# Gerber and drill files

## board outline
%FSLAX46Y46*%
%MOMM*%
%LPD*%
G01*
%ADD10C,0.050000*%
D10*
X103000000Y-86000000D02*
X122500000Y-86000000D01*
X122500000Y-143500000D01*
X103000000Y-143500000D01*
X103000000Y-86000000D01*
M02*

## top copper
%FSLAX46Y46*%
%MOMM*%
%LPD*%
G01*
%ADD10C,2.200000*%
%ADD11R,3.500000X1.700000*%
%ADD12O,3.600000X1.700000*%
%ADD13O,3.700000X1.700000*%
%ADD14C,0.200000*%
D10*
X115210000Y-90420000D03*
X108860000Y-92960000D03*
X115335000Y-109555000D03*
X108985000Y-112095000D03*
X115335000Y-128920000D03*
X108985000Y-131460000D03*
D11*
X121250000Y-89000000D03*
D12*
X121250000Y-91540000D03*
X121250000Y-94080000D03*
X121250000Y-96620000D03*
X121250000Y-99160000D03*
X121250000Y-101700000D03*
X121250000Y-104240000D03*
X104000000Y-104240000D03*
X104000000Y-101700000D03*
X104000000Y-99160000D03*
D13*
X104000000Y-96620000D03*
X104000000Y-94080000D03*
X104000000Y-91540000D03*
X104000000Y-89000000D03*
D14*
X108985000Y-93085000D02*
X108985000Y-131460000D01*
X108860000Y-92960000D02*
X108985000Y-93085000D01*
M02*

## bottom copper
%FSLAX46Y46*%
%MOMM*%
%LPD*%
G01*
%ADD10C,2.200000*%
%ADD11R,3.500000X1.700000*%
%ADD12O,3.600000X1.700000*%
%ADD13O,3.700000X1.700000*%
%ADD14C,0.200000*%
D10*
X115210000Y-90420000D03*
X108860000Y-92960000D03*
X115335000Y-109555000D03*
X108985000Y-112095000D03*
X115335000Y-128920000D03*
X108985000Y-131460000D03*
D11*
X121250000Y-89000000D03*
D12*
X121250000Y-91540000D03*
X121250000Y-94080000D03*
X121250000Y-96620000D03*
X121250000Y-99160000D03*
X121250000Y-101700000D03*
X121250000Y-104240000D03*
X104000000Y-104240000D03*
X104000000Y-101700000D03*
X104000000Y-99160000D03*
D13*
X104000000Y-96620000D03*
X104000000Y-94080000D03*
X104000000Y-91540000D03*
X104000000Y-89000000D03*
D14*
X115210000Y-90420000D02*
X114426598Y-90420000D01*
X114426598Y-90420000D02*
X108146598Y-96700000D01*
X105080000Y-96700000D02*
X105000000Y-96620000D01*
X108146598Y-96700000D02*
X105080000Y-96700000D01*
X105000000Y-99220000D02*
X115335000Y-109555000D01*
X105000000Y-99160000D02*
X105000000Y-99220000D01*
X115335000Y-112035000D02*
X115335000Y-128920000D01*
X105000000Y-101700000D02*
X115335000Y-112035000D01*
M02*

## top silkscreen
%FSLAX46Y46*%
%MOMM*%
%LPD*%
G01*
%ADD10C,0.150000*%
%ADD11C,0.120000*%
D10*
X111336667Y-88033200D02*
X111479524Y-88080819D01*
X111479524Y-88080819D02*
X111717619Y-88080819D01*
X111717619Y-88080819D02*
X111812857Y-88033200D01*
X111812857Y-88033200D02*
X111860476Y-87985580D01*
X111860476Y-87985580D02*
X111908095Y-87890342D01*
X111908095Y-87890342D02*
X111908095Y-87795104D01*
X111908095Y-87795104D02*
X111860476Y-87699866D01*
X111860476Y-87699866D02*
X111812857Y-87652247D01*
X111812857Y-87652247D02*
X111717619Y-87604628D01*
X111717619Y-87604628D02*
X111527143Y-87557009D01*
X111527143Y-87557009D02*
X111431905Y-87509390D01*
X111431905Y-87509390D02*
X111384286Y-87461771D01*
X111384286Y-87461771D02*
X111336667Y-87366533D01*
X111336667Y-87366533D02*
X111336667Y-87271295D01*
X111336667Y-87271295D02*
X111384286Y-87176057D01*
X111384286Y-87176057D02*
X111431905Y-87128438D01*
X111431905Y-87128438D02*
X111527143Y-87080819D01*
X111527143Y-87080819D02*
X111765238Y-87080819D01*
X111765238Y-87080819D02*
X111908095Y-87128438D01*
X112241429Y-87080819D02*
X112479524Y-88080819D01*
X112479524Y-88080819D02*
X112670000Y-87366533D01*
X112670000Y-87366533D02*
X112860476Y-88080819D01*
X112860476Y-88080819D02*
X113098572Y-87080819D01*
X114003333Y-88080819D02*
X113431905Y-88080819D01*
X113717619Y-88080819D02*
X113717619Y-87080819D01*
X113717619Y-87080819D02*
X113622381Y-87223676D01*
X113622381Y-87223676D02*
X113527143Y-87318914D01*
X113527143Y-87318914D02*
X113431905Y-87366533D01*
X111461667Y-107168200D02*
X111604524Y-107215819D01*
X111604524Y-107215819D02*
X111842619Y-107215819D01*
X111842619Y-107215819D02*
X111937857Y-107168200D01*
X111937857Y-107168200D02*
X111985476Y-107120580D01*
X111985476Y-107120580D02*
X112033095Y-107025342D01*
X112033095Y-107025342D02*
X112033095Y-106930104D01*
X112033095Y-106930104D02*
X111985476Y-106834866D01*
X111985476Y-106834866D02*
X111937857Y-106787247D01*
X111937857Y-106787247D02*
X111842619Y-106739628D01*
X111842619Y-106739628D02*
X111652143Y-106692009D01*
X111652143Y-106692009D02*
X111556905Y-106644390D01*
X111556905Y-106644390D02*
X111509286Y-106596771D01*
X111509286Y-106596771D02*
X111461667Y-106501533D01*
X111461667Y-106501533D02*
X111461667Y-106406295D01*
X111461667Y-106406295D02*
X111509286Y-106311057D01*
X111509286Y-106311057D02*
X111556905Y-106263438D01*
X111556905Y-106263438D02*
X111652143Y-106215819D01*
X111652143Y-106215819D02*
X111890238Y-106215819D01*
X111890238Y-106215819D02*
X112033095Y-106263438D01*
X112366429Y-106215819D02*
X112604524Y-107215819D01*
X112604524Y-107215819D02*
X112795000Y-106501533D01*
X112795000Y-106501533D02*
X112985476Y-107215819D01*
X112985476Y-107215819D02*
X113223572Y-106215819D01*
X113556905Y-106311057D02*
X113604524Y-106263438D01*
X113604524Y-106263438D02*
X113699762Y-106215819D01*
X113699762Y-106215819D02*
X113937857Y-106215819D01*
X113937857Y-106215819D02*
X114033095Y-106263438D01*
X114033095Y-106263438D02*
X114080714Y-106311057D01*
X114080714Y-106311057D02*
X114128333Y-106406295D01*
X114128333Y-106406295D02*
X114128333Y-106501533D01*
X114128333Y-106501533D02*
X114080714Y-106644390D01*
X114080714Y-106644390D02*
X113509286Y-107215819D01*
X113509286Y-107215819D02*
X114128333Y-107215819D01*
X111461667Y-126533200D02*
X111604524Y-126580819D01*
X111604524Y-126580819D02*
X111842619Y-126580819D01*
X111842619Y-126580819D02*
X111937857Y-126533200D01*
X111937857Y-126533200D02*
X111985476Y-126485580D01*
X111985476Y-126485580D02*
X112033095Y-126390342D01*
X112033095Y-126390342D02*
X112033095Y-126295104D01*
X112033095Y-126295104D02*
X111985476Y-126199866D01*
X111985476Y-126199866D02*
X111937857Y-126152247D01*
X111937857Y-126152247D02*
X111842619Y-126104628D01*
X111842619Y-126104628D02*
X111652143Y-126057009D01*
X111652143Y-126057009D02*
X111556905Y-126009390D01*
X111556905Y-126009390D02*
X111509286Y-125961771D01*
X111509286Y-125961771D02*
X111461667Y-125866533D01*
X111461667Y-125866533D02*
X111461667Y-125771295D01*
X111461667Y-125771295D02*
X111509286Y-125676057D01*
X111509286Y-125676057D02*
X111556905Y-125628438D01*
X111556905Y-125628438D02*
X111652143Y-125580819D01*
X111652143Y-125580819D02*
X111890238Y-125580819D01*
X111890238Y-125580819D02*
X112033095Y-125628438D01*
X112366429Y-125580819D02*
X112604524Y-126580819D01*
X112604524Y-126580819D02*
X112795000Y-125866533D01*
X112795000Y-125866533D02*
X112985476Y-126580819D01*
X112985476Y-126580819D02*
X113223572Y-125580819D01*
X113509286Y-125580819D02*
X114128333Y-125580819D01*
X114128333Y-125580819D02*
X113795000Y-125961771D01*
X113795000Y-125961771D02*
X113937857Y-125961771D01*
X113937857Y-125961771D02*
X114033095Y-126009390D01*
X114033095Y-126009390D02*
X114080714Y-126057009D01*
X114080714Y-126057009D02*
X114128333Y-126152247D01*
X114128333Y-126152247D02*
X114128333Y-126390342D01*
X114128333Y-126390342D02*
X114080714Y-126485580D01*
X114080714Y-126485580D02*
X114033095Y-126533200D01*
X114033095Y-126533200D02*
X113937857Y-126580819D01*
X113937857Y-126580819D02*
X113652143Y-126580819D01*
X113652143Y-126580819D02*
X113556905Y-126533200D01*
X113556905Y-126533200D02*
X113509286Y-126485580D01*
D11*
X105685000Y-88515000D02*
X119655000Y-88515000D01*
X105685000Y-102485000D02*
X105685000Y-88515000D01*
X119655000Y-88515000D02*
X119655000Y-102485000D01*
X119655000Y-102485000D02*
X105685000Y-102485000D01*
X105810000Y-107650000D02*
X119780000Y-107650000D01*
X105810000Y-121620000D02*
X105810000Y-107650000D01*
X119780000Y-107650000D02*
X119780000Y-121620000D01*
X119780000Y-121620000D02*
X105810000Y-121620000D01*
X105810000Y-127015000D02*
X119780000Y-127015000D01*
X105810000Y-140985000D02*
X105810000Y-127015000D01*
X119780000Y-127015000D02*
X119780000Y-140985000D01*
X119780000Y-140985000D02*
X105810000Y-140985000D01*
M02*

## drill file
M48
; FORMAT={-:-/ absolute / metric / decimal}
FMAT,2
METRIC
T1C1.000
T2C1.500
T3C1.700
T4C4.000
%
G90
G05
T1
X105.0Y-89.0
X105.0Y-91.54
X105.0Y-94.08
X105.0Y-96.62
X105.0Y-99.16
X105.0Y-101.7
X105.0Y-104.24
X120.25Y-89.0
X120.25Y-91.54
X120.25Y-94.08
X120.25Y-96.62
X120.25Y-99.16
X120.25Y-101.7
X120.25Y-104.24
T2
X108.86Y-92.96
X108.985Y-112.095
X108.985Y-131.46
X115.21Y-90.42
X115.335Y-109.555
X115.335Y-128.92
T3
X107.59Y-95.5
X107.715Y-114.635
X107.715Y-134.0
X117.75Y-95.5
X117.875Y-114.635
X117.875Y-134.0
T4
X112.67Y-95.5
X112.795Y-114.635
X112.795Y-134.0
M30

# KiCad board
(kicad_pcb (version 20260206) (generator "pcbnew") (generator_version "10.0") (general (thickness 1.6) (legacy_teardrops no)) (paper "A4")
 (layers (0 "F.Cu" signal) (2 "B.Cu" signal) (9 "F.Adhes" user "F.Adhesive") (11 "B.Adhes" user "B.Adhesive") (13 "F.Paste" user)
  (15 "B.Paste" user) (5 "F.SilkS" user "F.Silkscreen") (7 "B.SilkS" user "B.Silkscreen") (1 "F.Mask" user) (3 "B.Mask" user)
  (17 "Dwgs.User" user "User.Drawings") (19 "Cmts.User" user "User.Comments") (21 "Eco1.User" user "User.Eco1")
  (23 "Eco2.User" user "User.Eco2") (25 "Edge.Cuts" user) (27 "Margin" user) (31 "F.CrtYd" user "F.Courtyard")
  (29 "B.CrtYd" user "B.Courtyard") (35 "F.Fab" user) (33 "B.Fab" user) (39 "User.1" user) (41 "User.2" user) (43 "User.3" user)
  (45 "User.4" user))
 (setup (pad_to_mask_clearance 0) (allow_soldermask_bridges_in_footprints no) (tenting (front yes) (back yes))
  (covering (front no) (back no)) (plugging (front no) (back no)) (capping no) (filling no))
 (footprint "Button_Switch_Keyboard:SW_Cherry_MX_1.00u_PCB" (layer "F.Cu") (at 115.21 90.42)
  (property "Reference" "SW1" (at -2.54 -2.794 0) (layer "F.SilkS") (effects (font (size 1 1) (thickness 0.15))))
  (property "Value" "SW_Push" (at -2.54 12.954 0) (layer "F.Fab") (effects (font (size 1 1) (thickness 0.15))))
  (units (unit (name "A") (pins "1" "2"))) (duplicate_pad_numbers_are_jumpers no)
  (fp_line (start -9.525 -1.905) (end 4.445 -1.905) (stroke (width 0.12) (type solid)) (layer "F.SilkS"))
  (fp_line (start -9.525 12.065) (end -9.525 -1.905) (stroke (width 0.12) (type solid)) (layer "F.SilkS"))
  (fp_line (start 4.445 -1.905) (end 4.445 12.065) (stroke (width 0.12) (type solid)) (layer "F.SilkS"))
  (fp_line (start 4.445 12.065) (end -9.525 12.065) (stroke (width 0.12) (type solid)) (layer "F.SilkS"))
  (pad "" np_thru_hole circle (at -7.62 5.08) (size 1.7 1.7) (drill 1.7) (layers "*.Cu" "*.Mask"))
  (pad "" np_thru_hole circle (at -2.54 5.08) (size 4 4) (drill 4) (layers "*.Cu" "*.Mask"))
  (pad "" np_thru_hole circle (at 2.54 5.08) (size 1.7 1.7) (drill 1.7) (layers "*.Cu" "*.Mask"))
  (pad "1" thru_hole circle (at 0 0) (size 2.2 2.2) (drill 1.5) (layers "*.Cu" "*.Mask") (remove_unused_layers no)
   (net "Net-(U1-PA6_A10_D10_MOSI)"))
  (pad "2" thru_hole circle (at -6.35 2.54) (size 2.2 2.2) (drill 1.5) (layers "*.Cu" "*.Mask") (remove_unused_layers no) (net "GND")))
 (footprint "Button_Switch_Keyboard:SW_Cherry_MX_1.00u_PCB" (layer "F.Cu") (at 115.335 109.555)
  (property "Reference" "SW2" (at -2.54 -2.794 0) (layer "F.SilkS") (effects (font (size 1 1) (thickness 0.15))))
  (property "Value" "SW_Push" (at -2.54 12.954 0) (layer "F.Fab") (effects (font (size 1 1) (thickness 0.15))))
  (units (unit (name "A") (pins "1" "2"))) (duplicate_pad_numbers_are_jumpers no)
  (fp_line (start -9.525 -1.905) (end 4.445 -1.905) (stroke (width 0.12) (type solid)) (layer "F.SilkS"))
  (fp_line (start -9.525 12.065) (end -9.525 -1.905) (stroke (width 0.12) (type solid)) (layer "F.SilkS"))
  (fp_line (start 4.445 -1.905) (end 4.445 12.065) (stroke (width 0.12) (type solid)) (layer "F.SilkS"))
  (fp_line (start 4.445 12.065) (end -9.525 12.065) (stroke (width 0.12) (type solid)) (layer "F.SilkS"))
  (pad "" np_thru_hole circle (at -7.62 5.08) (size 1.7 1.7) (drill 1.7) (layers "*.Cu" "*.Mask"))
  (pad "" np_thru_hole circle (at -2.54 5.08) (size 4 4) (drill 4) (layers "*.Cu" "*.Mask"))
  (pad "" np_thru_hole circle (at 2.54 5.08) (size 1.7 1.7) (drill 1.7) (layers "*.Cu" "*.Mask"))
  (pad "1" thru_hole circle (at 0 0) (size 2.2 2.2) (drill 1.5) (layers "*.Cu" "*.Mask") (remove_unused_layers no)
   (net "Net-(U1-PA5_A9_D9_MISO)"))
  (pad "2" thru_hole circle (at -6.35 2.54) (size 2.2 2.2) (drill 1.5) (layers "*.Cu" "*.Mask") (remove_unused_layers no) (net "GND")))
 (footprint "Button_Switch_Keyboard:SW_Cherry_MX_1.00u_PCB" (layer "F.Cu") (at 115.335 128.92)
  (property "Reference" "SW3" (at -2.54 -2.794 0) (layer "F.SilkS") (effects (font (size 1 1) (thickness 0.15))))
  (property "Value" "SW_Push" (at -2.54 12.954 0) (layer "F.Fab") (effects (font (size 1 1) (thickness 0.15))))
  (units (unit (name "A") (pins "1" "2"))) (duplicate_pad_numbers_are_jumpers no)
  (fp_line (start -9.525 -1.905) (end 4.445 -1.905) (stroke (width 0.12) (type solid)) (layer "F.SilkS"))
  (fp_line (start -9.525 12.065) (end -9.525 -1.905) (stroke (width 0.12) (type solid)) (layer "F.SilkS"))
  (fp_line (start 4.445 -1.905) (end 4.445 12.065) (stroke (width 0.12) (type solid)) (layer "F.SilkS"))
  (fp_line (start 4.445 12.065) (end -9.525 12.065) (stroke (width 0.12) (type solid)) (layer "F.SilkS"))
  (pad "" np_thru_hole circle (at -7.62 5.08) (size 1.7 1.7) (drill 1.7) (layers "*.Cu" "*.Mask"))
  (pad "" np_thru_hole circle (at -2.54 5.08) (size 4 4) (drill 4) (layers "*.Cu" "*.Mask"))
  (pad "" np_thru_hole circle (at 2.54 5.08) (size 1.7 1.7) (drill 1.7) (layers "*.Cu" "*.Mask"))
  (pad "1" thru_hole circle (at 0 0) (size 2.2 2.2) (drill 1.5) (layers "*.Cu" "*.Mask") (remove_unused_layers no)
   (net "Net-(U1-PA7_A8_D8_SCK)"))
  (pad "2" thru_hole circle (at -6.35 2.54) (size 2.2 2.2) (drill 1.5) (layers "*.Cu" "*.Mask") (remove_unused_layers no) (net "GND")))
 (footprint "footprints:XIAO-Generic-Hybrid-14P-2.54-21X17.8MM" (layer "B.Cu") (at 112.625 96.62 180)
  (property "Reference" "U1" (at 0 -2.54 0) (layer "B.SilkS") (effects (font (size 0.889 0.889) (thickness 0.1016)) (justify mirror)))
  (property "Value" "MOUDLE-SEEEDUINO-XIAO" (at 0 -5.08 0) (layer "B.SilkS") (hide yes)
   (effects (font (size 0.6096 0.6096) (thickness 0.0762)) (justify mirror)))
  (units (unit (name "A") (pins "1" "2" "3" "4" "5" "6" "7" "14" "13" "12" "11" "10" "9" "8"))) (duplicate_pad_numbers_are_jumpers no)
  (pad "1" thru_hole rect (at -7.625 7.62 180) (size 3.5 1.7) (drill 1 (offset -1 0)) (layers "*.Cu" "*.Mask") (remove_unused_layers no)
   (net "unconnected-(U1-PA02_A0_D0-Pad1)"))
  (pad "2" thru_hole oval (at -7.625 5.08 180) (size 3.6 1.7) (drill 1 (offset -1 0)) (layers "*.Cu" "*.Mask") (remove_unused_layers no)
   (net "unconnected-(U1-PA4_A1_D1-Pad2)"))
  (pad "3" thru_hole oval (at -7.625 2.54 180) (size 3.6 1.7) (drill 1 (offset -1 0)) (layers "*.Cu" "*.Mask") (remove_unused_layers no)
   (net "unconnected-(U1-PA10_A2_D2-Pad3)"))
  (pad "4" thru_hole oval (at -7.625 0 180) (size 3.6 1.7) (drill 1 (offset -1 0)) (layers "*.Cu" "*.Mask") (remove_unused_layers no)
   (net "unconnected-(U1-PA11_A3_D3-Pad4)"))
  (pad "5" thru_hole oval (at -7.625 -2.54 180) (size 3.6 1.7) (drill 1 (offset -1 0)) (layers "*.Cu" "*.Mask") (remove_unused_layers no)
   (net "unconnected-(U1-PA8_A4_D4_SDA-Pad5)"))
  (pad "6" thru_hole oval (at -7.625 -5.08) (size 3.6 1.7) (drill 1 (offset 1 0)) (layers "*.Cu" "*.Mask") (remove_unused_layers no)
   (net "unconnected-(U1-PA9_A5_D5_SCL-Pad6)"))
  (pad "7" thru_hole oval (at -7.625 -7.62 180) (size 3.6 1.7) (drill 1 (offset -1 0)) (layers "*.Cu" "*.Mask") (remove_unused_layers no)
   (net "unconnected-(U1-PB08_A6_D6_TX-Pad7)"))
  (pad "8" thru_hole oval (at 7.625 -7.62 180) (size 3.6 1.7) (drill 1 (offset 1 0)) (layers "*.Cu" "*.Mask") (remove_unused_layers no)
   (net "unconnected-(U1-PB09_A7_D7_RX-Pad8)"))
  (pad "9" thru_hole oval (at 7.625 -5.08 180) (size 3.6 1.7) (drill 1 (offset 1 0)) (layers "*.Cu" "*.Mask") (remove_unused_layers no)
   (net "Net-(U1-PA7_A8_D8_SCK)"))
  (pad "10" thru_hole oval (at 7.625 -2.54 180) (size 3.6 1.7) (drill 1 (offset 1 0)) (layers "*.Cu" "*.Mask") (remove_unused_layers no)
   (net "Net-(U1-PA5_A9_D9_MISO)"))
  (pad "11" thru_hole oval (at 7.625 0 180) (size 3.7 1.7) (drill 1 (offset 1 0)) (layers "*.Cu" "*.Mask") (remove_unused_layers no)
   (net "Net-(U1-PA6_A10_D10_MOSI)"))
  (pad "12" thru_hole oval (at 7.625 2.54 180) (size 3.7 1.7) (drill 1 (offset 1 0)) (layers "*.Cu" "*.Mask") (remove_unused_layers no)
   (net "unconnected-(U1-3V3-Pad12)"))
  (pad "13" thru_hole oval (at 7.625 5.08 180) (size 3.7 1.7) (drill 1 (offset 1 0)) (layers "*.Cu" "*.Mask") (remove_unused_layers no)
   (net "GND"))
  (pad "14" thru_hole oval (at 7.625 7.62 180) (size 3.7 1.7) (drill 1 (offset 1 0)) (layers "*.Cu" "*.Mask") (remove_unused_layers no)
   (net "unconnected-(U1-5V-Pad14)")))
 (gr_rect (start 103 86) (end 122.5 143.5) (stroke (width 0.05) (type default)) (fill no) (layer "Edge.Cuts"))
 (segment (start 108.985 93.085) (end 108.985 131.46) (width 0.2) (layer "F.Cu") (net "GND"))
 (segment (start 108.86 92.96) (end 108.985 93.085) (width 0.2) (layer "F.Cu") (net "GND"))
 (segment (start 115.21 90.42) (end 114.426598 90.42) (width 0.2) (layer "B.Cu") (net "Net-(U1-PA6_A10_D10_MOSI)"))
 (segment (start 114.426598 90.42) (end 108.146598 96.7) (width 0.2) (layer "B.Cu") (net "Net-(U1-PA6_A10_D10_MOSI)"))
 (segment (start 105.08 96.7) (end 105 96.62) (width 0.2) (layer "B.Cu") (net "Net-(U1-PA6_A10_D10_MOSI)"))
 (segment (start 108.146598 96.7) (end 105.08 96.7) (width 0.2) (layer "B.Cu") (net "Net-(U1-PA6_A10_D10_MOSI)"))
 (segment (start 105 99.22) (end 115.335 109.555) (width 0.2) (layer "B.Cu") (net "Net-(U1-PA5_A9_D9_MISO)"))
 (segment (start 105 99.16) (end 105 99.22) (width 0.2) (layer "B.Cu") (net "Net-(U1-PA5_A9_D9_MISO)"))
 (segment (start 115.335 112.035) (end 115.335 128.92) (width 0.2) (layer "B.Cu") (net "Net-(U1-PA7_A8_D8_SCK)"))
 (segment (start 105 101.7) (end 115.335 112.035) (width 0.2) (layer "B.Cu") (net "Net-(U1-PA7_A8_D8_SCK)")))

